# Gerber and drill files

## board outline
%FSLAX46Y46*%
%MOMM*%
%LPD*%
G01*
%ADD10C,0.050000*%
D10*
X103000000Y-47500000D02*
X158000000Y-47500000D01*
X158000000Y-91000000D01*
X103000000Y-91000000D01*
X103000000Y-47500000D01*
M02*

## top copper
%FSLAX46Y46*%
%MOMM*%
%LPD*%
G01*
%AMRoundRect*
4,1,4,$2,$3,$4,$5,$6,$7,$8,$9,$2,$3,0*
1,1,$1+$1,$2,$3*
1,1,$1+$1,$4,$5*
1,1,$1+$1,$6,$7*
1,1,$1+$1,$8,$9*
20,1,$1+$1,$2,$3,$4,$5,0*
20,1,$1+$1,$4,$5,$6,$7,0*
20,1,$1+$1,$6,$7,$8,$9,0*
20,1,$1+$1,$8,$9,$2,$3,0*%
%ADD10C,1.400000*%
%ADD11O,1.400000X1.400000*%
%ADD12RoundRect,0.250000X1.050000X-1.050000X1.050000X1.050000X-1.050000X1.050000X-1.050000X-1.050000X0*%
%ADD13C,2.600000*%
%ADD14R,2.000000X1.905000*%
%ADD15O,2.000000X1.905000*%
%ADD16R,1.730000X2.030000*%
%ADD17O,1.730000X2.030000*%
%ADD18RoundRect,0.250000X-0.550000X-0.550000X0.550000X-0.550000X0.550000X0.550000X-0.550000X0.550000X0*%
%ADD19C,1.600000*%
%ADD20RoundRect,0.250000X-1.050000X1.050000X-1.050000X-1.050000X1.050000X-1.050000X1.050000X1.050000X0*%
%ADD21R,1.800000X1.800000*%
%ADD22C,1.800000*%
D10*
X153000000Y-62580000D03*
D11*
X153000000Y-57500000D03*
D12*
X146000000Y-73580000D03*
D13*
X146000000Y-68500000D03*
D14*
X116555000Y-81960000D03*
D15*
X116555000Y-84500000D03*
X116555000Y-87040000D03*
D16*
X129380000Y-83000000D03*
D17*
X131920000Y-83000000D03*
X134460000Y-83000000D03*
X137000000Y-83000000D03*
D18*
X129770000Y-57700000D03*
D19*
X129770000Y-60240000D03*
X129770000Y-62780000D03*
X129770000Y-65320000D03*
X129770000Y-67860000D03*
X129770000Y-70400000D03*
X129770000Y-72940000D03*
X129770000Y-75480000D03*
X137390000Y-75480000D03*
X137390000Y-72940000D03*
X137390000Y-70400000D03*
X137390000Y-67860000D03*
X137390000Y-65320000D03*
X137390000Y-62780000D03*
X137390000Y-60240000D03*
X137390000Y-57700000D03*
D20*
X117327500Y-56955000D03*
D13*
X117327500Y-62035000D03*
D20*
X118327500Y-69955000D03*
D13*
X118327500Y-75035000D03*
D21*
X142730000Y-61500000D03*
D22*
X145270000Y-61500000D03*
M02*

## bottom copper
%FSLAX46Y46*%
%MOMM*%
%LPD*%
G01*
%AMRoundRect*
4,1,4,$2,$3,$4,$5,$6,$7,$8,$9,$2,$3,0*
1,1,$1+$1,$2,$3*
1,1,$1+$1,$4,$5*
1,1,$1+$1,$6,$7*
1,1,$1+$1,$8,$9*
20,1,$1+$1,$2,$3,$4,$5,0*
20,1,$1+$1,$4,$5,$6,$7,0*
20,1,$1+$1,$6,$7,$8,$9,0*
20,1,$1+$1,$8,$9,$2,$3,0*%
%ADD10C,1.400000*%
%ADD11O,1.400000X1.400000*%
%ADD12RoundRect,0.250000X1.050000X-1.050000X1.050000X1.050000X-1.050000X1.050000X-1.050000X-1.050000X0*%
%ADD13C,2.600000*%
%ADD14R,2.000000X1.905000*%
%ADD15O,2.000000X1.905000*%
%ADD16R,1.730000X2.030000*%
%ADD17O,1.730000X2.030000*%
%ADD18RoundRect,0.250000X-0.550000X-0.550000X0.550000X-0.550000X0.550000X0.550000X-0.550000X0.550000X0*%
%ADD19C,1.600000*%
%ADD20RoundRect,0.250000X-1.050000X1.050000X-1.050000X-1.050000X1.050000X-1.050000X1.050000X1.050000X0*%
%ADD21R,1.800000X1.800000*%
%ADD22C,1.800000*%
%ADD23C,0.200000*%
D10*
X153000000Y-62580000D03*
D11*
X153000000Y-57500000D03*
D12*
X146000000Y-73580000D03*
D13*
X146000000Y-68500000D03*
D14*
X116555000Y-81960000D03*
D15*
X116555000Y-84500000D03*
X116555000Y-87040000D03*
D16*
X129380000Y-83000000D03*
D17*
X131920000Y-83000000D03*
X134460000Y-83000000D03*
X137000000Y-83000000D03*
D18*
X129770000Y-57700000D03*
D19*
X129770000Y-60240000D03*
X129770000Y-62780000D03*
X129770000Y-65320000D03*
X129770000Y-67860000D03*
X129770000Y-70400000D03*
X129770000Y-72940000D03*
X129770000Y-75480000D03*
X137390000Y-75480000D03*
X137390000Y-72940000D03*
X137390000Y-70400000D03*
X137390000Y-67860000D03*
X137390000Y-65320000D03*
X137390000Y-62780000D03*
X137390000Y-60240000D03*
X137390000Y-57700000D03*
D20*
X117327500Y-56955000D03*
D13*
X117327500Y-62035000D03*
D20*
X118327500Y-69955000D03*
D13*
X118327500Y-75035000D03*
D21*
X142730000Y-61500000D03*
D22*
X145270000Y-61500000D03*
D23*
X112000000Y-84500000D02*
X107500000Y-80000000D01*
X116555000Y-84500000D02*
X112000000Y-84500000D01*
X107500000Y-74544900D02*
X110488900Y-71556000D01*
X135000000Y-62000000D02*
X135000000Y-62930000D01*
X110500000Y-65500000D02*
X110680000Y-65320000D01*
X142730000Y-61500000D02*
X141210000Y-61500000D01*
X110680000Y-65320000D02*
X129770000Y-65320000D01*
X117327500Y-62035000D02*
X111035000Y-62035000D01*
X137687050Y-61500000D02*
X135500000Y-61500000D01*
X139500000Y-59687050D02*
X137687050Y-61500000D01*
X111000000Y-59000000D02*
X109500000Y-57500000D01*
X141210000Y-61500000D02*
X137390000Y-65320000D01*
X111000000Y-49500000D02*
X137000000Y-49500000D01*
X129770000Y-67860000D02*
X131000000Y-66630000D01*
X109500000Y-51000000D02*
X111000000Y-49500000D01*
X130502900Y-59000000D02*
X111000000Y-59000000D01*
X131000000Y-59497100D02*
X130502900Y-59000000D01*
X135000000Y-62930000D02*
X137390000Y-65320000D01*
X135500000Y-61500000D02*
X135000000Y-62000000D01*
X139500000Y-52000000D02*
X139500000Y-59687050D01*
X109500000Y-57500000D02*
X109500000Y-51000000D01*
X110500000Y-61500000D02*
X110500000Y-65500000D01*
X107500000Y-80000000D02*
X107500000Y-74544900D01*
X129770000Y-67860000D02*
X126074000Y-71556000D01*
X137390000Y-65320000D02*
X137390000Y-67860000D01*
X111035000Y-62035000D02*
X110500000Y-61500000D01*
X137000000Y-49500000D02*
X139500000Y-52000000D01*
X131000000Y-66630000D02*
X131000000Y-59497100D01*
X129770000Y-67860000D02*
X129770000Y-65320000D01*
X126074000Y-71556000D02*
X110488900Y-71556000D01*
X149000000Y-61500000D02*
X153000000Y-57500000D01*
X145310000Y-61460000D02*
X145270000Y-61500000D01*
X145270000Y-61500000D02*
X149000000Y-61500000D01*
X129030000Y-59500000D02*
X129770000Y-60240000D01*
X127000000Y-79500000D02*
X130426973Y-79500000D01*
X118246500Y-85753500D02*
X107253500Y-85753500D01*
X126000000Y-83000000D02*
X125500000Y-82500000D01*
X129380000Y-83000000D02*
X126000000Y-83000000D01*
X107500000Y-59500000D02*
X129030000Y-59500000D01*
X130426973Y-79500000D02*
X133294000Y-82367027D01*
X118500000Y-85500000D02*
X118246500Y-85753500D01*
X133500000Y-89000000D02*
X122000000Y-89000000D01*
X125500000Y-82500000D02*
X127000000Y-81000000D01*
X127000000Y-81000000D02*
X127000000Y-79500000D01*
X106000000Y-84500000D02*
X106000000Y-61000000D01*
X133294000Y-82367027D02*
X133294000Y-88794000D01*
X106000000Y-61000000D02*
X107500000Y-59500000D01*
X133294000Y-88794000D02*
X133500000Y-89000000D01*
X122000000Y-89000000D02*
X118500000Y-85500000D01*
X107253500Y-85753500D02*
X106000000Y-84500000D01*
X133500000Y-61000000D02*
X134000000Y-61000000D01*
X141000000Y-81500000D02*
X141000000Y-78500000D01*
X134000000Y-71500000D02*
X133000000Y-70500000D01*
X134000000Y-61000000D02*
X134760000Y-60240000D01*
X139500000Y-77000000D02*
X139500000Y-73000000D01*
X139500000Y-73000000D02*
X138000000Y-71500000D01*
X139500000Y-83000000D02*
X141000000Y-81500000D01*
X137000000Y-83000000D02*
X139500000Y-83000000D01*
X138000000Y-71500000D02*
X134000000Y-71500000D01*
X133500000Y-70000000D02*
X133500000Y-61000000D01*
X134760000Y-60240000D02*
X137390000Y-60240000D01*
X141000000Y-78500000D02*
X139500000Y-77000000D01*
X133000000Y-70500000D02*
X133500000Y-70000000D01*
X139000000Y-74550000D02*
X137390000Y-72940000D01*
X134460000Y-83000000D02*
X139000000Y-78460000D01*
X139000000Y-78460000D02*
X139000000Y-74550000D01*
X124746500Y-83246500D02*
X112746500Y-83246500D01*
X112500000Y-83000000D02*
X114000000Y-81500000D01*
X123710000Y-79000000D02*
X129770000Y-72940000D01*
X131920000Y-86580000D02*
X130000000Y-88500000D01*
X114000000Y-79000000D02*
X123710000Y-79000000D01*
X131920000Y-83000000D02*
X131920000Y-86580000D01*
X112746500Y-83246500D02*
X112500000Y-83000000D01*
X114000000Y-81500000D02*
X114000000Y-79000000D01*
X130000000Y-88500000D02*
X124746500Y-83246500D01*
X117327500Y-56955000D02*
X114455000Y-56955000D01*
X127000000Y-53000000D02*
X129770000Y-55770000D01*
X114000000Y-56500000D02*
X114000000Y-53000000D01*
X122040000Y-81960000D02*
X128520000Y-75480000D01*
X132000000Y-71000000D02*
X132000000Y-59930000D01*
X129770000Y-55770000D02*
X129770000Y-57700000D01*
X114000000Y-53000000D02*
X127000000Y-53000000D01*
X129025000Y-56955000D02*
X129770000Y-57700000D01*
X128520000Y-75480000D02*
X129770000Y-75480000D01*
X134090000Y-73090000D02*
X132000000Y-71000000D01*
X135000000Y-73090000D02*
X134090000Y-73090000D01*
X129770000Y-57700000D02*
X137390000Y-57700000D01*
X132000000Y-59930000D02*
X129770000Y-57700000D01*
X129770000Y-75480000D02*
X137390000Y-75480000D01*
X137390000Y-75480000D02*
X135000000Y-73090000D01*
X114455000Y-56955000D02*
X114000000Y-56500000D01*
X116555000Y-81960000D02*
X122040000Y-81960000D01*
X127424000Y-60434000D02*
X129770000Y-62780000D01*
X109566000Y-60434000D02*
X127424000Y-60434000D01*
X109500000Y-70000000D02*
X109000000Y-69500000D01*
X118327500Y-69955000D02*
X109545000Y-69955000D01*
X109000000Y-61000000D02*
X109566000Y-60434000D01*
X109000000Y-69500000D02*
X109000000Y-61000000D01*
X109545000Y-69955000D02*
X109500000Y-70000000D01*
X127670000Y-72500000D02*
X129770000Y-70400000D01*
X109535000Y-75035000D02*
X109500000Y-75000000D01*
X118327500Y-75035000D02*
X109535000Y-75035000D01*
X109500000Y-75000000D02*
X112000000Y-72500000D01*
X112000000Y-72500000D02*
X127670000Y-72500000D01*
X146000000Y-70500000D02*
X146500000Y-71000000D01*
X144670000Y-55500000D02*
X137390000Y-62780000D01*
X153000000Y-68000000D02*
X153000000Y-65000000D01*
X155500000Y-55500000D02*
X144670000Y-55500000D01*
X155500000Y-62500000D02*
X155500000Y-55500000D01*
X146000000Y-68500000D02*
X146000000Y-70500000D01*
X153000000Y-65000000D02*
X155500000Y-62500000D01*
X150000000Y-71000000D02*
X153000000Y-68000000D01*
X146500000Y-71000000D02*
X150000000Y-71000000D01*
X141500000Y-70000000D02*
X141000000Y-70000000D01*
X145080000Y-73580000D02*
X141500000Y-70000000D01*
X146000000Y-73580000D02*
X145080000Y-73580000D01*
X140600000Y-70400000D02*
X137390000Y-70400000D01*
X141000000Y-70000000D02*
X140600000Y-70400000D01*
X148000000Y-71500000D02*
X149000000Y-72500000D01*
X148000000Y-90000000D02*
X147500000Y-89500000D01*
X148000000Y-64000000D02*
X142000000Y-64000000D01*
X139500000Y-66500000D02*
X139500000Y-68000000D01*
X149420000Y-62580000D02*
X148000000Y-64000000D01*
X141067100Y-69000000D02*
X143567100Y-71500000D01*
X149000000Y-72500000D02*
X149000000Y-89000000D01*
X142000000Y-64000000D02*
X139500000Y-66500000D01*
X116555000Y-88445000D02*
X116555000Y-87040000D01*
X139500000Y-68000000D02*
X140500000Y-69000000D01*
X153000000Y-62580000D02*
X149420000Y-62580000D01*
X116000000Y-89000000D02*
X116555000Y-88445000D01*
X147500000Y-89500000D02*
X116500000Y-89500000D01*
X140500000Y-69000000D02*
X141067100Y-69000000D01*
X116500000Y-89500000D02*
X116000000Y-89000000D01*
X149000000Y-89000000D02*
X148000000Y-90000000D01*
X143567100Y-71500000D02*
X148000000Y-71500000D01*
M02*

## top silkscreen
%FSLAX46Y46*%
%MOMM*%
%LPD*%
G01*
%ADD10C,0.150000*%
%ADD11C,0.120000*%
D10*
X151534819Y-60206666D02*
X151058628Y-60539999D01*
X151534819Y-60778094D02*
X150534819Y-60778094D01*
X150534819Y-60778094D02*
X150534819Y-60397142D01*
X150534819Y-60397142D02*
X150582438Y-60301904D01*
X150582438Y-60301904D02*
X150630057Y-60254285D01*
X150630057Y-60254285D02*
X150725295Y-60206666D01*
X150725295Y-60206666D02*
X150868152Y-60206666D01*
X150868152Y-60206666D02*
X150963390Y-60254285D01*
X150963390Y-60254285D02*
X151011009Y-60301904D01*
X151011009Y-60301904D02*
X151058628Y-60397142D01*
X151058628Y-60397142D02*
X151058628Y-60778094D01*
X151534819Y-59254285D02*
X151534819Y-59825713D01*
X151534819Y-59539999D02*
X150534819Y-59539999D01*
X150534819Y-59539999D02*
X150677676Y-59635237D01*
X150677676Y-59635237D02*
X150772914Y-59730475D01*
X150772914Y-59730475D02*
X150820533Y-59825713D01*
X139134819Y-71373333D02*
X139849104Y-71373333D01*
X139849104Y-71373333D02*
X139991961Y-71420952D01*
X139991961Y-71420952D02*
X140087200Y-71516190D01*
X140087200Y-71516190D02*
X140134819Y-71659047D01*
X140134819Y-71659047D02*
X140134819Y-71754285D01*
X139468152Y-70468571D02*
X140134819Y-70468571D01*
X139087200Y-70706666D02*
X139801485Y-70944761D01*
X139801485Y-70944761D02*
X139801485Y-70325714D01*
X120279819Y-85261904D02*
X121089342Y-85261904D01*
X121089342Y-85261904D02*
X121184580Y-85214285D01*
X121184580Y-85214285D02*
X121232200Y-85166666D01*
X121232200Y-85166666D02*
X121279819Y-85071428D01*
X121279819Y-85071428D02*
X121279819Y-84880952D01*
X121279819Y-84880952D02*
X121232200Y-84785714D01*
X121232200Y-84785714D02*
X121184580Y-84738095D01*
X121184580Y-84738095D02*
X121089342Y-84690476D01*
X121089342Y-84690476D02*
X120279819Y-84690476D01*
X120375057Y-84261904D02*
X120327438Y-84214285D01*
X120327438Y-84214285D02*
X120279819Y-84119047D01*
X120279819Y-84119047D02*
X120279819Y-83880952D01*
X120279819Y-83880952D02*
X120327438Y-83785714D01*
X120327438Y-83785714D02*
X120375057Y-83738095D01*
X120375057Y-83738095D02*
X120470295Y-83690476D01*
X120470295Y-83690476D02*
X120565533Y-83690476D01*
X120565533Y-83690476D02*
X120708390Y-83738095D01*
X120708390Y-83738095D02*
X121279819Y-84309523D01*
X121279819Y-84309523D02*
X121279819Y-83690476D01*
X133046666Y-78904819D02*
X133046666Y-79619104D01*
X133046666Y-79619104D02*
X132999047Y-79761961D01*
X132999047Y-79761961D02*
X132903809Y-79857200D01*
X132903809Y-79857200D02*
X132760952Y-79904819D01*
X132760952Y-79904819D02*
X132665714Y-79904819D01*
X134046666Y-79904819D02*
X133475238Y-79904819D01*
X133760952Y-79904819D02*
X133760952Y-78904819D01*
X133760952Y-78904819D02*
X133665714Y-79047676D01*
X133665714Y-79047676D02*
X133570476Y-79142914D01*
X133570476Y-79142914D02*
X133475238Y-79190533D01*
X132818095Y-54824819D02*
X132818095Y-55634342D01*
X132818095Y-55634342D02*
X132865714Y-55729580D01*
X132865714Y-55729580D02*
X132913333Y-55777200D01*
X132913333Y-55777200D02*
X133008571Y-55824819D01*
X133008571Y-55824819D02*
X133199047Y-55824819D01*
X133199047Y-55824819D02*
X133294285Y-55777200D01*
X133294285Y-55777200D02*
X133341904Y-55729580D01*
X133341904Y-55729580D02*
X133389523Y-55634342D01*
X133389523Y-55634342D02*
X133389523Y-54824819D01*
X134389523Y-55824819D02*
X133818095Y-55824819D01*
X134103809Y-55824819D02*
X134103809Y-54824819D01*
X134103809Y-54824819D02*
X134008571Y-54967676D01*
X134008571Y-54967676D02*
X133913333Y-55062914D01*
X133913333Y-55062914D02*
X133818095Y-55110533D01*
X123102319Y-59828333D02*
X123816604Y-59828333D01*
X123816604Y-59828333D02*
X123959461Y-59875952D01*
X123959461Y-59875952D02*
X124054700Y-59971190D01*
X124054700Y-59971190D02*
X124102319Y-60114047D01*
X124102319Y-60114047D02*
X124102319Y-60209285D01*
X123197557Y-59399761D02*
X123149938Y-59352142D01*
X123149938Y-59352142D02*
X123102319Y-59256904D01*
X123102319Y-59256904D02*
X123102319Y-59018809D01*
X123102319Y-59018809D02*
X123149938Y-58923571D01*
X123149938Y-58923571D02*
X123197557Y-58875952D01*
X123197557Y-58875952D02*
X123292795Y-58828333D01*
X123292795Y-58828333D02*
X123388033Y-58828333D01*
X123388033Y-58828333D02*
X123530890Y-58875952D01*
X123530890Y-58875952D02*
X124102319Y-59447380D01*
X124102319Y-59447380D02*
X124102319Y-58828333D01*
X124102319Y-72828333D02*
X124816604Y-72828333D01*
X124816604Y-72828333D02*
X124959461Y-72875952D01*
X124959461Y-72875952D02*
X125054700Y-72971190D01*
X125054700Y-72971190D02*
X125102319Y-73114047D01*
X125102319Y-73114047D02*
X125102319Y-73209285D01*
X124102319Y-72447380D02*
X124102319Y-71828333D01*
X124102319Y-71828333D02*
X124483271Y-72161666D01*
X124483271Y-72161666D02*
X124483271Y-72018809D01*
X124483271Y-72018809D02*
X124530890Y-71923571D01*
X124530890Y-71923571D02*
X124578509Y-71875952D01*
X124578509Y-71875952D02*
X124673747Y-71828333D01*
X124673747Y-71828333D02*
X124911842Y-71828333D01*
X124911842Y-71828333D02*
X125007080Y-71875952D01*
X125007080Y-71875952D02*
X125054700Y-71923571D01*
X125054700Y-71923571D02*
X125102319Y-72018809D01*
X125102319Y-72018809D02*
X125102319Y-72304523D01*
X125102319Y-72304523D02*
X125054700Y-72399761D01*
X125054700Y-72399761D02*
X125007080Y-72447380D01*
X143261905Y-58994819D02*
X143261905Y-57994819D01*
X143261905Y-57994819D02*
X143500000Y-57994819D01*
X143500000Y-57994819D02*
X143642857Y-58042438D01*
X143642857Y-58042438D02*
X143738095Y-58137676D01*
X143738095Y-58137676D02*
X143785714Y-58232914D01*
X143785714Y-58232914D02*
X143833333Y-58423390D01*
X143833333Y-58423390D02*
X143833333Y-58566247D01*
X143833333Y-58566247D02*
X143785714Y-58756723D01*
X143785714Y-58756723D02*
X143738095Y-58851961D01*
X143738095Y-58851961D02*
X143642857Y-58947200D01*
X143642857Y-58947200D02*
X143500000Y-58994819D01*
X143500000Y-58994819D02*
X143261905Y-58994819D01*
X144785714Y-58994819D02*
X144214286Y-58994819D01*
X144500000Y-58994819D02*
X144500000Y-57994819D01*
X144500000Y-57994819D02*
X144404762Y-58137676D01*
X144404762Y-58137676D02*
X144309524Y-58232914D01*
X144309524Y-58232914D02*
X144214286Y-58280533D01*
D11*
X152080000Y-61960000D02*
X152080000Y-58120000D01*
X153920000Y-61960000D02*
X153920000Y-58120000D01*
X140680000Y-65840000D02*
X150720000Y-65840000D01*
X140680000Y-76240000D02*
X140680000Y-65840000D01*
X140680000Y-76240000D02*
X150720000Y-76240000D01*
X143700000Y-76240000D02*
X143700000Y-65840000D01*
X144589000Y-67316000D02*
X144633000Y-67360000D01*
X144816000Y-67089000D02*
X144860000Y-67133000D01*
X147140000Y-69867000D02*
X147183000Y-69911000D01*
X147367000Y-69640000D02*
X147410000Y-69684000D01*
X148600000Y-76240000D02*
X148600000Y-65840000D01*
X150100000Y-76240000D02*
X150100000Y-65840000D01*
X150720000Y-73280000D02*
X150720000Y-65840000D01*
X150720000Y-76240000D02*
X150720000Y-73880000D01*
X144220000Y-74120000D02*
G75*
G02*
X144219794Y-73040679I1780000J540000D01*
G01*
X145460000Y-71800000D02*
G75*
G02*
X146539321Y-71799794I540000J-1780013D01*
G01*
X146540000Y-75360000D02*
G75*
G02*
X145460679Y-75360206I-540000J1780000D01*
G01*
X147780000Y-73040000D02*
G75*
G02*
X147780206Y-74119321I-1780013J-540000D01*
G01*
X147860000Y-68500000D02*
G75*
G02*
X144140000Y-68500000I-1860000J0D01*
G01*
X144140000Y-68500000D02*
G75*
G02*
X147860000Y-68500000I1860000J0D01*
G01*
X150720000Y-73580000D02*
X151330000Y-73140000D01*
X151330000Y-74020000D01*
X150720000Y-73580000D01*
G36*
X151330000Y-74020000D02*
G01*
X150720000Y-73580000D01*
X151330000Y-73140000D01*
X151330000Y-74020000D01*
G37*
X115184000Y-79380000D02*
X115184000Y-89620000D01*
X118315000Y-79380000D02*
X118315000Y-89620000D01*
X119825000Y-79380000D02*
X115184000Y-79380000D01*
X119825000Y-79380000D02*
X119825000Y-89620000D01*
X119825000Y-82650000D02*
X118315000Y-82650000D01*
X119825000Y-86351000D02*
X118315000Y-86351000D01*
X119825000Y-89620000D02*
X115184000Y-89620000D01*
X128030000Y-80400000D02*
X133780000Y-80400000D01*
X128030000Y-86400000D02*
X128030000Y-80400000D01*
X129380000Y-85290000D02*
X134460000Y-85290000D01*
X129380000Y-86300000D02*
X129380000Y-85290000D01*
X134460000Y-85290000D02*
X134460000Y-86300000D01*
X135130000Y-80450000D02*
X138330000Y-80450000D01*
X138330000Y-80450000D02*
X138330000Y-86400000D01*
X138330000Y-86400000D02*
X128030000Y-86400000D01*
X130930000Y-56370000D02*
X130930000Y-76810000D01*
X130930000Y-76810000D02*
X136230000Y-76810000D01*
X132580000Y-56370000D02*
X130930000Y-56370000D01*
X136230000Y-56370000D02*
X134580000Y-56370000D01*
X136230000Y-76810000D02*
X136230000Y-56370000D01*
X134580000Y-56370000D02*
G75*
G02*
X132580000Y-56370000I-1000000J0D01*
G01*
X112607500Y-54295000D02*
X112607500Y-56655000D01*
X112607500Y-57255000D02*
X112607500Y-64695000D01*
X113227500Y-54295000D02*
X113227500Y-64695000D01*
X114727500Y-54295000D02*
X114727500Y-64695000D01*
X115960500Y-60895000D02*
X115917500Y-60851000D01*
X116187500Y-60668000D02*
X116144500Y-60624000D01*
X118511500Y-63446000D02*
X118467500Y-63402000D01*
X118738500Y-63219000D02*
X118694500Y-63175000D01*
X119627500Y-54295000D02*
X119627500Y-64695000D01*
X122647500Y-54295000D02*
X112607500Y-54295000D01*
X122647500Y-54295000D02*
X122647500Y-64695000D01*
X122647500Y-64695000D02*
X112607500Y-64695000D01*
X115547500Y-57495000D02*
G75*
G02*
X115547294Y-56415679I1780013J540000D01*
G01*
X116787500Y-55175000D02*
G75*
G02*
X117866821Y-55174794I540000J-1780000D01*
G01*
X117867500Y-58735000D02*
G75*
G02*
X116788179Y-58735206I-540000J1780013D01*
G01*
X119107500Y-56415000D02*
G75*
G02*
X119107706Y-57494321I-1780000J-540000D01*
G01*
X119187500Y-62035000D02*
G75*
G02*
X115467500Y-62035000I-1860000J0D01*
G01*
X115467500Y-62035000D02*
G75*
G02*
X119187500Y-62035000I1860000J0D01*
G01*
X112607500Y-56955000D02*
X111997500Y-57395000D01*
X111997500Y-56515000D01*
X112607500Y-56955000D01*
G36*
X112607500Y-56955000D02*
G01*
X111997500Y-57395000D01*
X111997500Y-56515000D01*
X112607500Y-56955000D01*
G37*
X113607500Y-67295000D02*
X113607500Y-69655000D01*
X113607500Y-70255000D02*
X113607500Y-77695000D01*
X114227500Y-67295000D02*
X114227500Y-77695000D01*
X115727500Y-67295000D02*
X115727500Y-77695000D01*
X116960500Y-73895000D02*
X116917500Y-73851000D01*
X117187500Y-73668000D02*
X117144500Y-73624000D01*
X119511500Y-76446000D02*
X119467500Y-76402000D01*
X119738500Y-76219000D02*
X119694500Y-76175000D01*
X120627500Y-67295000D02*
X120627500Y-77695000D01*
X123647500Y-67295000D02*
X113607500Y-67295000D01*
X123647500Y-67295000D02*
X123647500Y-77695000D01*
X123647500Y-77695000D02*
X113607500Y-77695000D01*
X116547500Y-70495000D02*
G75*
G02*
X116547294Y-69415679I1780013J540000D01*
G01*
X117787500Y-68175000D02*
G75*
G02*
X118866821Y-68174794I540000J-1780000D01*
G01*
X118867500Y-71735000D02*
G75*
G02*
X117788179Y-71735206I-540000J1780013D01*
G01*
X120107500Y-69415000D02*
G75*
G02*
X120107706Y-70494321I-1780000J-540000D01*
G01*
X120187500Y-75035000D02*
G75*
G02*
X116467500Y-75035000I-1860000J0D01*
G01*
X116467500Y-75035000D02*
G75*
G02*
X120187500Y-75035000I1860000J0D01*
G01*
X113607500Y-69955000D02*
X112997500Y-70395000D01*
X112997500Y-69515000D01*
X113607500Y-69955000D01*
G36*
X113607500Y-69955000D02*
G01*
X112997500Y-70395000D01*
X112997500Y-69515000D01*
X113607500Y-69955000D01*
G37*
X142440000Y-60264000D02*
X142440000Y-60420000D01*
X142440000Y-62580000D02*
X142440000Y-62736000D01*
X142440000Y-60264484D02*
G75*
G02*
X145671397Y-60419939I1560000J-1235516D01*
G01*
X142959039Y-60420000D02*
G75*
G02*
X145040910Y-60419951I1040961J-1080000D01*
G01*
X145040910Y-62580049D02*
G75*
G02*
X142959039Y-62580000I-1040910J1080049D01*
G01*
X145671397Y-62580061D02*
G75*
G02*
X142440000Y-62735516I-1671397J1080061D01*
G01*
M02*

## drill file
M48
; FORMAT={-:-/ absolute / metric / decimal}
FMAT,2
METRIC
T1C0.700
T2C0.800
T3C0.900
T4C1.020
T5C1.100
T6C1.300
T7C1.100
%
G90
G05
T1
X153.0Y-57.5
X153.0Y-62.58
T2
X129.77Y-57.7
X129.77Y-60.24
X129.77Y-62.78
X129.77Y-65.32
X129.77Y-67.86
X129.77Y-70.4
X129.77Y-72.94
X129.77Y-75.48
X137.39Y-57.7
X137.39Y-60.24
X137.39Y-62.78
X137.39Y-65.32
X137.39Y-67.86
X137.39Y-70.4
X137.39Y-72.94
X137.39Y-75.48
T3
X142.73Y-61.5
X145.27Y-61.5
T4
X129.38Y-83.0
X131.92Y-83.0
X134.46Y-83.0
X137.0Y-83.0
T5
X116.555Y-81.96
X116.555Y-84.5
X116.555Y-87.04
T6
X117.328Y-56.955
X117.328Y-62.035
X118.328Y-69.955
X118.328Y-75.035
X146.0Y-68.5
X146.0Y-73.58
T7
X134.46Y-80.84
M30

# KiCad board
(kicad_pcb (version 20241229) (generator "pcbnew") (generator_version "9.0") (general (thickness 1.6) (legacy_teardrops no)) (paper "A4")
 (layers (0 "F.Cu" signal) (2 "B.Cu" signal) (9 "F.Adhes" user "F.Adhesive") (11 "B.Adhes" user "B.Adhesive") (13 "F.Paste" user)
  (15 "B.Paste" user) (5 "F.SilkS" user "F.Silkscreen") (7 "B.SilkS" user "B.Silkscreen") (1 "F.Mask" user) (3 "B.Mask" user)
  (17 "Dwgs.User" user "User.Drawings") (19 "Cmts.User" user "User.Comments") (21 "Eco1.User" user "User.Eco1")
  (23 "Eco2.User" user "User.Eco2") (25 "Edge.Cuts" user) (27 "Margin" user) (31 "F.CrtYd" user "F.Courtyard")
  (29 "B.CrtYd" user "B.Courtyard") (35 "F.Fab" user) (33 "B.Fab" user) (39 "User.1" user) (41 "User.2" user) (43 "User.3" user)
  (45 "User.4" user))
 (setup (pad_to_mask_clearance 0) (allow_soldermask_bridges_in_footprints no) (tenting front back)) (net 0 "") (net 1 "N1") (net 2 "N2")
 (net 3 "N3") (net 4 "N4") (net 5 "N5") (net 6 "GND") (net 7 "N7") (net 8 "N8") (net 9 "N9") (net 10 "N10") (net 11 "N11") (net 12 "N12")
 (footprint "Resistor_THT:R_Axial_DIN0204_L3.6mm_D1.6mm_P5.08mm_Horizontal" (layer "F.Cu") (at 153 62.58 90)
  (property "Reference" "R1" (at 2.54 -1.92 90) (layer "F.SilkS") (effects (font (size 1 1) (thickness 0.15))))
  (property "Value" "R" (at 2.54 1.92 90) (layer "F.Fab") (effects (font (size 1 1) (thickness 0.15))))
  (fp_line (start 0.62 -0.92) (end 4.46 -0.92) (stroke (width 0.12) (type solid)) (layer "F.SilkS"))
  (fp_line (start 0.62 0.92) (end 4.46 0.92) (stroke (width 0.12) (type solid)) (layer "F.SilkS"))
  (pad "1" thru_hole circle (at 0 0 90) (size 1.4 1.4) (drill 0.7) (layers "*.Cu" "*.Mask") (remove_unused_layers no) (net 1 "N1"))
  (pad "2" thru_hole oval (at 5.08 0 90) (size 1.4 1.4) (drill 0.7) (layers "*.Cu" "*.Mask") (remove_unused_layers no) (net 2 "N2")))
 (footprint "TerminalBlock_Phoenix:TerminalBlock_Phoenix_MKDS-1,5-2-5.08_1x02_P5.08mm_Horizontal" (layer "F.Cu") (at 146 73.58 90)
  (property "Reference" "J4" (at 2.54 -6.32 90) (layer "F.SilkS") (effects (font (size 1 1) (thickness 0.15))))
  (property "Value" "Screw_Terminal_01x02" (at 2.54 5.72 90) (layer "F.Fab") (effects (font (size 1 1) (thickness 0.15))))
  (fp_line (start 7.74 -5.32) (end 7.74 4.72) (stroke (width 0.12) (type solid)) (layer "F.SilkS"))
  (fp_line (start -2.66 -5.32) (end 7.74 -5.32) (stroke (width 0.12) (type solid)) (layer "F.SilkS"))
  (fp_line (start -2.66 -5.32) (end -2.66 4.72) (stroke (width 0.12) (type solid)) (layer "F.SilkS"))
  (fp_line (start -2.66 -2.3) (end 7.74 -2.3) (stroke (width 0.12) (type solid)) (layer "F.SilkS"))
  (fp_line (start 6.264 -1.411) (end 6.22 -1.367) (stroke (width 0.12) (type solid)) (layer "F.SilkS"))
  (fp_line (start 6.491 -1.184) (end 6.447 -1.14) (stroke (width 0.12) (type solid)) (layer "F.SilkS"))
  (fp_line (start 3.713 1.14) (end 3.669 1.183) (stroke (width 0.12) (type solid)) (layer "F.SilkS"))
  (fp_line (start 3.94 1.367) (end 3.896 1.41) (stroke (width 0.12) (type solid)) (layer "F.SilkS"))
  (fp_line (start -2.66 2.6) (end 7.74 2.6) (stroke (width 0.12) (type solid)) (layer "F.SilkS"))
  (fp_line (start -2.66 4.1) (end 7.74 4.1) (stroke (width 0.12) (type solid)) (layer "F.SilkS"))
  (fp_line (start 0.3 4.72) (end 7.74 4.72) (stroke (width 0.12) (type solid)) (layer "F.SilkS"))
  (fp_line (start -2.66 4.72) (end -0.3 4.72) (stroke (width 0.12) (type solid)) (layer "F.SilkS"))
  (fp_arc (start -0.54 -1.78) (mid -0.000355 -1.860107) (end 0.539321 -1.780206) (stroke (width 0.12) (type solid)) (layer "F.SilkS"))
  (fp_arc (start 1.78 -0.54) (mid 1.860107 -0.000355) (end 1.780206 0.539321) (stroke (width 0.12) (type solid)) (layer "F.SilkS"))
  (fp_arc (start -1.78 0.54) (mid -1.860107 0.000355) (end -1.780206 -0.539321) (stroke (width 0.12) (type solid)) (layer "F.SilkS"))
  (fp_arc (start 0.54 1.78) (mid 0.000355 1.860107) (end -0.539321 1.780206) (stroke (width 0.12) (type solid)) (layer "F.SilkS"))
  (fp_circle (center 5.08 0) (end 6.94 0) (stroke (width 0.12) (type solid)) (fill no) (layer "F.SilkS"))
  (fp_poly (pts (xy 0 4.72) (xy 0.44 5.33) (xy -0.44 5.33) (xy 0 4.72)) (stroke (width 0.12) (type solid)) (fill yes) (layer "F.SilkS"))
  (pad "1" thru_hole roundrect (at 0 0 90) (size 2.6 2.6) (drill 1.3) (layers "*.Cu" "*.Mask") (remove_unused_layers no)
   (roundrect_rratio 0.096154) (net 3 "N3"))
  (pad "2" thru_hole circle (at 5.08 0 90) (size 2.6 2.6) (drill 1.3) (layers "*.Cu" "*.Mask") (remove_unused_layers no) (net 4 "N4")))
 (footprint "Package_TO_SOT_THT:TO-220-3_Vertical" (layer "F.Cu") (at 116.555 81.96 -90)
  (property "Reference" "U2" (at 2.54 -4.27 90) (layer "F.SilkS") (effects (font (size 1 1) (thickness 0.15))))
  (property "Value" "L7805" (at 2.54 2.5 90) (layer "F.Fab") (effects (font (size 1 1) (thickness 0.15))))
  (fp_line (start -2.58 1.371) (end 7.66 1.371) (stroke (width 0.12) (type solid)) (layer "F.SilkS"))
  (fp_line (start -2.58 -1.76) (end 7.66 -1.76) (stroke (width 0.12) (type solid)) (layer "F.SilkS"))
  (fp_line (start -2.58 -3.27) (end -2.58 1.371) (stroke (width 0.12) (type solid)) (layer "F.SilkS"))
  (fp_line (start -2.58 -3.27) (end 7.66 -3.27) (stroke (width 0.12) (type solid)) (layer "F.SilkS"))
  (fp_line (start 0.69 -3.27) (end 0.69 -1.76) (stroke (width 0.12) (type solid)) (layer "F.SilkS"))
  (fp_line (start 4.391 -3.27) (end 4.391 -1.76) (stroke (width 0.12) (type solid)) (layer "F.SilkS"))
  (fp_line (start 7.66 -3.27) (end 7.66 1.371) (stroke (width 0.12) (type solid)) (layer "F.SilkS"))
  (pad "1" thru_hole rect (at 0 0 270) (size 1.905 2) (drill 1.1) (layers "*.Cu" "*.Mask") (remove_unused_layers no) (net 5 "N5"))
  (pad "2" thru_hole oval (at 2.54 0 270) (size 1.905 2) (drill 1.1) (layers "*.Cu" "*.Mask") (remove_unused_layers no) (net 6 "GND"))
  (pad "3" thru_hole oval (at 5.08 0 270) (size 1.905 2) (drill 1.1) (layers "*.Cu" "*.Mask") (remove_unused_layers no) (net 1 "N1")))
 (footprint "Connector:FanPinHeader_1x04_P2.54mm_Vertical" (layer "F.Cu") (at 129.38 83)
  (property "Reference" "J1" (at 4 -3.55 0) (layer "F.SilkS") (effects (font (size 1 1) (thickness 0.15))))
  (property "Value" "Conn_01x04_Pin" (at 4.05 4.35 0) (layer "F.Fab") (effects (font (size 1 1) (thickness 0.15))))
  (fp_line (start -1.35 -2.6) (end 4.4 -2.6) (stroke (width 0.12) (type solid)) (layer "F.SilkS"))
  (fp_line (start -1.35 3.4) (end -1.35 -2.6) (stroke (width 0.12) (type solid)) (layer "F.SilkS"))
  (fp_line (start 0 2.29) (end 5.08 2.29) (stroke (width 0.12) (type solid)) (layer "F.SilkS"))
  (fp_line (start 0 3.3) (end 0 2.29) (stroke (width 0.12) (type solid)) (layer "F.SilkS"))
  (fp_line (start 5.08 2.29) (end 5.08 3.3) (stroke (width 0.12) (type solid)) (layer "F.SilkS"))
  (fp_line (start 5.75 -2.55) (end 8.95 -2.55) (stroke (width 0.12) (type solid)) (layer "F.SilkS"))
  (fp_line (start 8.95 -2.55) (end 8.95 3.4) (stroke (width 0.12) (type solid)) (layer "F.SilkS"))
  (fp_line (start 8.95 3.4) (end -1.35 3.4) (stroke (width 0.12) (type solid)) (layer "F.SilkS"))
  (pad "" np_thru_hole circle (at 5.08 -2.16 90) (size 1.1 1.1) (drill 1.1) (layers "*.Cu" "*.Mask"))
  (pad "1" thru_hole rect (at 0 0 90) (size 2.03 1.73) (drill 1.02) (layers "*.Cu" "*.Mask") (remove_unused_layers no) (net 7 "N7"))
  (pad "2" thru_hole oval (at 2.54 0 90) (size 2.03 1.73) (drill 1.02) (layers "*.Cu" "*.Mask") (remove_unused_layers no) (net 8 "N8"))
  (pad "3" thru_hole oval (at 5.08 0 90) (size 2.03 1.73) (drill 1.02) (layers "*.Cu" "*.Mask") (remove_unused_layers no) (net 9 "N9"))
  (pad "4" thru_hole oval (at 7.62 0 90) (size 2.03 1.73) (drill 1.02) (layers "*.Cu" "*.Mask") (remove_unused_layers no) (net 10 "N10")))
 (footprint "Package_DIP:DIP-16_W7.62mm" (layer "F.Cu") (at 129.77 57.7)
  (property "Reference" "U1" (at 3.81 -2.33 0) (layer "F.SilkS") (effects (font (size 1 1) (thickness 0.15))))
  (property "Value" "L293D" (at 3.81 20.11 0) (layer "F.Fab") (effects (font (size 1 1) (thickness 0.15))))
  (fp_line (start 1.16 -1.33) (end 1.16 19.11) (stroke (width 0.12) (type solid)) (layer "F.SilkS"))
  (fp_line (start 1.16 19.11) (end 6.46 19.11) (stroke (width 0.12) (type solid)) (layer "F.SilkS"))
  (fp_line (start 2.81 -1.33) (end 1.16 -1.33) (stroke (width 0.12) (type solid)) (layer "F.SilkS"))
  (fp_line (start 6.46 -1.33) (end 4.81 -1.33) (stroke (width 0.12) (type solid)) (layer "F.SilkS"))
  (fp_line (start 6.46 19.11) (end 6.46 -1.33) (stroke (width 0.12) (type solid)) (layer "F.SilkS"))
  (fp_arc (start 4.81 -1.33) (mid 3.81 -0.33) (end 2.81 -1.33) (stroke (width 0.12) (type solid)) (layer "F.SilkS"))
  (pad "1" thru_hole roundrect (at 0 0) (size 1.6 1.6) (drill 0.8) (layers "*.Cu" "*.Mask") (remove_unused_layers no)
   (roundrect_rratio 0.15625) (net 5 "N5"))
  (pad "2" thru_hole circle (at 0 2.54) (size 1.6 1.6) (drill 0.8) (layers "*.Cu" "*.Mask") (remove_unused_layers no) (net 7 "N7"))
  (pad "3" thru_hole circle (at 0 5.08) (size 1.6 1.6) (drill 0.8) (layers "*.Cu" "*.Mask") (remove_unused_layers no) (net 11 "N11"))
  (pad "4" thru_hole circle (at 0 7.62) (size 1.6 1.6) (drill 0.8) (layers "*.Cu" "*.Mask") (remove_unused_layers no) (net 6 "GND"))
  (pad "5" thru_hole circle (at 0 10.16) (size 1.6 1.6) (drill 0.8) (layers "*.Cu" "*.Mask") (remove_unused_layers no) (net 6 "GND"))
  (pad "6" thru_hole circle (at 0 12.7) (size 1.6 1.6) (drill 0.8) (layers "*.Cu" "*.Mask") (remove_unused_layers no) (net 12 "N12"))
  (pad "7" thru_hole circle (at 0 15.24) (size 1.6 1.6) (drill 0.8) (layers "*.Cu" "*.Mask") (remove_unused_layers no) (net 8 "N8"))
  (pad "8" thru_hole circle (at 0 17.78) (size 1.6 1.6) (drill 0.8) (layers "*.Cu" "*.Mask") (remove_unused_layers no) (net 5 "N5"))
  (pad "9" thru_hole circle (at 7.62 17.78) (size 1.6 1.6) (drill 0.8) (layers "*.Cu" "*.Mask") (remove_unused_layers no) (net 5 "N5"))
  (pad "10" thru_hole circle (at 7.62 15.24) (size 1.6 1.6) (drill 0.8) (layers "*.Cu" "*.Mask") (remove_unused_layers no) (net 9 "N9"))
  (pad "11" thru_hole circle (at 7.62 12.7) (size 1.6 1.6) (drill 0.8) (layers "*.Cu" "*.Mask") (remove_unused_layers no) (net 3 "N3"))
  (pad "12" thru_hole circle (at 7.62 10.16) (size 1.6 1.6) (drill 0.8) (layers "*.Cu" "*.Mask") (remove_unused_layers no) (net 6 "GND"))
  (pad "13" thru_hole circle (at 7.62 7.62) (size 1.6 1.6) (drill 0.8) (layers "*.Cu" "*.Mask") (remove_unused_layers no) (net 6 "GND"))
  (pad "14" thru_hole circle (at 7.62 5.08) (size 1.6 1.6) (drill 0.8) (layers "*.Cu" "*.Mask") (remove_unused_layers no) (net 4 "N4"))
  (pad "15" thru_hole circle (at 7.62 2.54) (size 1.6 1.6) (drill 0.8) (layers "*.Cu" "*.Mask") (remove_unused_layers no) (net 10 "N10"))
  (pad "16" thru_hole circle (at 7.62 0) (size 1.6 1.6) (drill 0.8) (layers "*.Cu" "*.Mask") (remove_unused_layers no) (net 5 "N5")))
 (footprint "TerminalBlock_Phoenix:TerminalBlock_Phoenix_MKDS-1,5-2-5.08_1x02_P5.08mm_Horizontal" (layer "F.Cu") (at 117.3275 56.955 -90)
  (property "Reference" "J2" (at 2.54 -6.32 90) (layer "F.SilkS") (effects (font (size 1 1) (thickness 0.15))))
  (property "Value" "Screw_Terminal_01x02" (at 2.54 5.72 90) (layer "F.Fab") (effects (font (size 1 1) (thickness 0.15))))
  (fp_line (start -2.66 4.72) (end -0.3 4.72) (stroke (width 0.12) (type solid)) (layer "F.SilkS"))
  (fp_line (start 0.3 4.72) (end 7.74 4.72) (stroke (width 0.12) (type solid)) (layer "F.SilkS"))
  (fp_line (start -2.66 4.1) (end 7.74 4.1) (stroke (width 0.12) (type solid)) (layer "F.SilkS"))
  (fp_line (start -2.66 2.6) (end 7.74 2.6) (stroke (width 0.12) (type solid)) (layer "F.SilkS"))
  (fp_line (start 3.94 1.367) (end 3.896 1.41) (stroke (width 0.12) (type solid)) (layer "F.SilkS"))
  (fp_line (start 3.713 1.14) (end 3.669 1.183) (stroke (width 0.12) (type solid)) (layer "F.SilkS"))
  (fp_line (start 6.491 -1.184) (end 6.447 -1.14) (stroke (width 0.12) (type solid)) (layer "F.SilkS"))
  (fp_line (start 6.264 -1.411) (end 6.22 -1.367) (stroke (width 0.12) (type solid)) (layer "F.SilkS"))
  (fp_line (start -2.66 -2.3) (end 7.74 -2.3) (stroke (width 0.12) (type solid)) (layer "F.SilkS"))
  (fp_line (start -2.66 -5.32) (end -2.66 4.72) (stroke (width 0.12) (type solid)) (layer "F.SilkS"))
  (fp_line (start -2.66 -5.32) (end 7.74 -5.32) (stroke (width 0.12) (type solid)) (layer "F.SilkS"))
  (fp_line (start 7.74 -5.32) (end 7.74 4.72) (stroke (width 0.12) (type solid)) (layer "F.SilkS"))
  (fp_arc (start 0.54 1.78) (mid 0.000355 1.860107) (end -0.539321 1.780206) (stroke (width 0.12) (type solid)) (layer "F.SilkS"))
  (fp_arc (start -1.78 0.54) (mid -1.860107 0.000355) (end -1.780206 -0.539321) (stroke (width 0.12) (type solid)) (layer "F.SilkS"))
  (fp_arc (start 1.78 -0.54) (mid 1.860107 -0.000355) (end 1.780206 0.539321) (stroke (width 0.12) (type solid)) (layer "F.SilkS"))
  (fp_arc (start -0.54 -1.78) (mid -0.000355 -1.860107) (end 0.539321 -1.780206) (stroke (width 0.12) (type solid)) (layer "F.SilkS"))
  (fp_circle (center 5.08 0) (end 6.94 0) (stroke (width 0.12) (type solid)) (fill no) (layer "F.SilkS"))
  (fp_poly (pts (xy 0 4.72) (xy 0.44 5.33) (xy -0.44 5.33) (xy 0 4.72)) (stroke (width 0.12) (type solid)) (fill yes) (layer "F.SilkS"))
  (pad "1" thru_hole roundrect (at 0 0 270) (size 2.6 2.6) (drill 1.3) (layers "*.Cu" "*.Mask") (remove_unused_layers no)
   (roundrect_rratio 0.096154) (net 5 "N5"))
  (pad "2" thru_hole circle (at 5.08 0 270) (size 2.6 2.6) (drill 1.3) (layers "*.Cu" "*.Mask") (remove_unused_layers no) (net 6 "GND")))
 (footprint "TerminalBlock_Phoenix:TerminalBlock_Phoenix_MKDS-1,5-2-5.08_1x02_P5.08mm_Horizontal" (layer "F.Cu") (at 118.3275 69.955 -90)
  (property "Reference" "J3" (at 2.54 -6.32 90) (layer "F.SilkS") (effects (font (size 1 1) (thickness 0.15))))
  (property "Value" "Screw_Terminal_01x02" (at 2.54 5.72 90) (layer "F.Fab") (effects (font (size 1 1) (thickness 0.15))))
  (fp_line (start -2.66 4.72) (end -0.3 4.72) (stroke (width 0.12) (type solid)) (layer "F.SilkS"))
  (fp_line (start 0.3 4.72) (end 7.74 4.72) (stroke (width 0.12) (type solid)) (layer "F.SilkS"))
  (fp_line (start -2.66 4.1) (end 7.74 4.1) (stroke (width 0.12) (type solid)) (layer "F.SilkS"))
  (fp_line (start -2.66 2.6) (end 7.74 2.6) (stroke (width 0.12) (type solid)) (layer "F.SilkS"))
  (fp_line (start 3.94 1.367) (end 3.896 1.41) (stroke (width 0.12) (type solid)) (layer "F.SilkS"))
  (fp_line (start 3.713 1.14) (end 3.669 1.183) (stroke (width 0.12) (type solid)) (layer "F.SilkS"))
  (fp_line (start 6.491 -1.184) (end 6.447 -1.14) (stroke (width 0.12) (type solid)) (layer "F.SilkS"))
  (fp_line (start 6.264 -1.411) (end 6.22 -1.367) (stroke (width 0.12) (type solid)) (layer "F.SilkS"))
  (fp_line (start -2.66 -2.3) (end 7.74 -2.3) (stroke (width 0.12) (type solid)) (layer "F.SilkS"))
  (fp_line (start -2.66 -5.32) (end -2.66 4.72) (stroke (width 0.12) (type solid)) (layer "F.SilkS"))
  (fp_line (start -2.66 -5.32) (end 7.74 -5.32) (stroke (width 0.12) (type solid)) (layer "F.SilkS"))
  (fp_line (start 7.74 -5.32) (end 7.74 4.72) (stroke (width 0.12) (type solid)) (layer "F.SilkS"))
  (fp_arc (start 0.54 1.78) (mid 0.000355 1.860107) (end -0.539321 1.780206) (stroke (width 0.12) (type solid)) (layer "F.SilkS"))
  (fp_arc (start -1.78 0.54) (mid -1.860107 0.000355) (end -1.780206 -0.539321) (stroke (width 0.12) (type solid)) (layer "F.SilkS"))
  (fp_arc (start 1.78 -0.54) (mid 1.860107 -0.000355) (end 1.780206 0.539321) (stroke (width 0.12) (type solid)) (layer "F.SilkS"))
  (fp_arc (start -0.54 -1.78) (mid -0.000355 -1.860107) (end 0.539321 -1.780206) (stroke (width 0.12) (type solid)) (layer "F.SilkS"))
  (fp_circle (center 5.08 0) (end 6.94 0) (stroke (width 0.12) (type solid)) (fill no) (layer "F.SilkS"))
  (fp_poly (pts (xy 0 4.72) (xy 0.44 5.33) (xy -0.44 5.33) (xy 0 4.72)) (stroke (width 0.12) (type solid)) (fill yes) (layer "F.SilkS"))
  (pad "1" thru_hole roundrect (at 0 0 270) (size 2.6 2.6) (drill 1.3) (layers "*.Cu" "*.Mask") (remove_unused_layers no)
   (roundrect_rratio 0.096154) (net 11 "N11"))
  (pad "2" thru_hole circle (at 5.08 0 270) (size 2.6 2.6) (drill 1.3) (layers "*.Cu" "*.Mask") (remove_unused_layers no) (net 12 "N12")))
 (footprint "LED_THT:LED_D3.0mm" (layer "F.Cu") (at 142.73 61.5)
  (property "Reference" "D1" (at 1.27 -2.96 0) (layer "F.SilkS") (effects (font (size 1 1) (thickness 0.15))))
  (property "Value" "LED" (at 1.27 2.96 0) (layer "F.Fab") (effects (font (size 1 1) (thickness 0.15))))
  (fp_line (start -0.29 -1.236) (end -0.29 -1.08) (stroke (width 0.12) (type solid)) (layer "F.SilkS"))
  (fp_line (start -0.29 1.08) (end -0.29 1.236) (stroke (width 0.12) (type solid)) (layer "F.SilkS"))
  (fp_arc (start -0.29 -1.235516) (mid 1.365624 -1.987701) (end 2.941397 -1.080061) (stroke (width 0.12) (type solid)) (layer "F.SilkS"))
  (fp_arc (start 0.229039 -1.08) (mid 1.269964 -1.5) (end 2.31091 -1.080049) (stroke (width 0.12) (type solid)) (layer "F.SilkS"))
  (fp_arc (start 2.31091 1.080049) (mid 1.269964 1.5) (end 0.229039 1.08) (stroke (width 0.12) (type solid)) (layer "F.SilkS"))
  (fp_arc (start 2.941397 1.080061) (mid 1.365624 1.987701) (end -0.29 1.235516) (stroke (width 0.12) (type solid)) (layer "F.SilkS"))
  (pad "1" thru_hole rect (at 0 0) (size 1.8 1.8) (drill 0.9) (layers "*.Cu" "*.Mask") (remove_unused_layers no) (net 6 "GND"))
  (pad "2" thru_hole circle (at 2.54 0) (size 1.8 1.8) (drill 0.9) (layers "*.Cu" "*.Mask") (remove_unused_layers no) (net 2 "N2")))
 (gr_rect (start 103 47.5) (end 158 91) (stroke (width 0.05) (type default)) (fill no) (layer "Edge.Cuts"))
 (segment (start 112 84.5) (end 107.5 80) (width 0.2) (layer "B.Cu") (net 6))
 (segment (start 116.555 84.5) (end 112 84.5) (width 0.2) (layer "B.Cu") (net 6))
 (segment (start 107.5 74.5449) (end 110.4889 71.556) (width 0.2) (layer "B.Cu") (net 6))
 (segment (start 135 62) (end 135 62.93) (width 0.2) (layer "B.Cu") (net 6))
 (segment (start 110.5 65.5) (end 110.68 65.32) (width 0.2) (layer "B.Cu") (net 6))
 (segment (start 142.73 61.5) (end 141.21 61.5) (width 0.2) (layer "B.Cu") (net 6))
 (segment (start 110.68 65.32) (end 129.77 65.32) (width 0.2) (layer "B.Cu") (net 6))
 (segment (start 117.3275 62.035) (end 111.035 62.035) (width 0.2) (layer "B.Cu") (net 6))
 (segment (start 137.68705 61.5) (end 135.5 61.5) (width 0.2) (layer "B.Cu") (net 6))
 (segment (start 139.5 59.68705) (end 137.68705 61.5) (width 0.2) (layer "B.Cu") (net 6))
 (segment (start 111 59) (end 109.5 57.5) (width 0.2) (layer "B.Cu") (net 6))
 (segment (start 141.21 61.5) (end 137.39 65.32) (width 0.2) (layer "B.Cu") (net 6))
 (segment (start 111 49.5) (end 137 49.5) (width 0.2) (layer "B.Cu") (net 6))
 (segment (start 129.77 67.86) (end 131 66.63) (width 0.2) (layer "B.Cu") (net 6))
 (segment (start 109.5 51) (end 111 49.5) (width 0.2) (layer "B.Cu") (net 6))
 (segment (start 130.5029 59) (end 111 59) (width 0.2) (layer "B.Cu") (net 6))
 (segment (start 131 59.4971) (end 130.5029 59) (width 0.2) (layer "B.Cu") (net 6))
 (segment (start 135 62.93) (end 137.39 65.32) (width 0.2) (layer "B.Cu") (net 6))
 (segment (start 135.5 61.5) (end 135 62) (width 0.2) (layer "B.Cu") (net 6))
 (segment (start 139.5 52) (end 139.5 59.68705) (width 0.2) (layer "B.Cu") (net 6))
 (segment (start 109.5 57.5) (end 109.5 51) (width 0.2) (layer "B.Cu") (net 6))
 (segment (start 110.5 61.5) (end 110.5 65.5) (width 0.2) (layer "B.Cu") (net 6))
 (segment (start 107.5 80) (end 107.5 74.5449) (width 0.2) (layer "B.Cu") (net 6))
 (segment (start 129.77 67.86) (end 126.074 71.556) (width 0.2) (layer "B.Cu") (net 6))
 (segment (start 137.39 65.32) (end 137.39 67.86) (width 0.2) (layer "B.Cu") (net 6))
 (segment (start 111.035 62.035) (end 110.5 61.5) (width 0.2) (layer "B.Cu") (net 6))
 (segment (start 137 49.5) (end 139.5 52) (width 0.2) (layer "B.Cu") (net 6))
 (segment (start 131 66.63) (end 131 59.4971) (width 0.2) (layer "B.Cu") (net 6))
 (segment (start 129.77 67.86) (end 129.77 65.32) (width 0.2) (layer "B.Cu") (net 6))
 (segment (start 126.074 71.556) (end 110.4889 71.556) (width 0.2) (layer "B.Cu") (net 6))
 (segment (start 149 61.5) (end 153 57.5) (width 0.2) (layer "B.Cu") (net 2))
 (segment (start 145.31 61.46) (end 145.27 61.5) (width 0.2) (layer "B.Cu") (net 2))
 (segment (start 145.27 61.5) (end 149 61.5) (width 0.2) (layer "B.Cu") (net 2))
 (segment (start 129.03 59.5) (end 129.77 60.24) (width 0.2) (layer "B.Cu") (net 7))
 (segment (start 127 79.5) (end 130.426973 79.5) (width 0.2) (layer "B.Cu") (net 7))
 (segment (start 118.2465 85.7535) (end 107.2535 85.7535) (width 0.2) (layer "B.Cu") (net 7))
 (segment (start 126 83) (end 125.5 82.5) (width 0.2) (layer "B.Cu") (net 7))
 (segment (start 129.38 83) (end 126 83) (width 0.2) (layer "B.Cu") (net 7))
 (segment (start 107.5 59.5) (end 129.03 59.5) (width 0.2) (layer "B.Cu") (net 7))
 (segment (start 130.426973 79.5) (end 133.294 82.367027) (width 0.2) (layer "B.Cu") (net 7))
 (segment (start 118.5 85.5) (end 118.2465 85.7535) (width 0.2) (layer "B.Cu") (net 7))
 (segment (start 133.5 89) (end 122 89) (width 0.2) (layer "B.Cu") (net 7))
 (segment (start 125.5 82.5) (end 127 81) (width 0.2) (layer "B.Cu") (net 7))
 (segment (start 127 81) (end 127 79.5) (width 0.2) (layer "B.Cu") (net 7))
 (segment (start 106 84.5) (end 106 61) (width 0.2) (layer "B.Cu") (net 7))
 (segment (start 133.294 82.367027) (end 133.294 88.794) (width 0.2) (layer "B.Cu") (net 7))
 (segment (start 106 61) (end 107.5 59.5) (width 0.2) (layer "B.Cu") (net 7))
 (segment (start 133.294 88.794) (end 133.5 89) (width 0.2) (layer "B.Cu") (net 7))
 (segment (start 122 89) (end 118.5 85.5) (width 0.2) (layer "B.Cu") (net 7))
 (segment (start 107.2535 85.7535) (end 106 84.5) (width 0.2) (layer "B.Cu") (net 7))
 (segment (start 133.5 61) (end 134 61) (width 0.2) (layer "B.Cu") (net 10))
 (segment (start 141 81.5) (end 141 78.5) (width 0.2) (layer "B.Cu") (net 10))
 (segment (start 134 71.5) (end 133 70.5) (width 0.2) (layer "B.Cu") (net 10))
 (segment (start 134 61) (end 134.76 60.24) (width 0.2) (layer "B.Cu") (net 10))
 (segment (start 139.5 77) (end 139.5 73) (width 0.2) (layer "B.Cu") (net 10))
 (segment (start 139.5 73) (end 138 71.5) (width 0.2) (layer "B.Cu") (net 10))
 (segment (start 139.5 83) (end 141 81.5) (width 0.2) (layer "B.Cu") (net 10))
 (segment (start 137 83) (end 139.5 83) (width 0.2) (layer "B.Cu") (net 10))
 (segment (start 138 71.5) (end 134 71.5) (width 0.2) (layer "B.Cu") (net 10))
 (segment (start 133.5 70) (end 133.5 61) (width 0.2) (layer "B.Cu") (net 10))
 (segment (start 134.76 60.24) (end 137.39 60.24) (width 0.2) (layer "B.Cu") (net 10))
 (segment (start 141 78.5) (end 139.5 77) (width 0.2) (layer "B.Cu") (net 10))
 (segment (start 133 70.5) (end 133.5 70) (width 0.2) (layer "B.Cu") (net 10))
 (segment (start 139 74.55) (end 137.39 72.94) (width 0.2) (layer "B.Cu") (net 9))
 (segment (start 134.46 83) (end 139 78.46) (width 0.2) (layer "B.Cu") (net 9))
 (segment (start 139 78.46) (end 139 74.55) (width 0.2) (layer "B.Cu") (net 9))
 (segment (start 124.7465 83.2465) (end 112.7465 83.2465) (width 0.2) (layer "B.Cu") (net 8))
 (segment (start 112.5 83) (end 114 81.5) (width 0.2) (layer "B.Cu") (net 8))
 (segment (start 123.71 79) (end 129.77 72.94) (width 0.2) (layer "B.Cu") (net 8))
 (segment (start 131.92 86.58) (end 130 88.5) (width 0.2) (layer "B.Cu") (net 8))
 (segment (start 114 79) (end 123.71 79) (width 0.2) (layer "B.Cu") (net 8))
 (segment (start 131.92 83) (end 131.92 86.58) (width 0.2) (layer "B.Cu") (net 8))
 (segment (start 112.7465 83.2465) (end 112.5 83) (width 0.2) (layer "B.Cu") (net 8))
 (segment (start 114 81.5) (end 114 79) (width 0.2) (layer "B.Cu") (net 8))
 (segment (start 130 88.5) (end 124.7465 83.2465) (width 0.2) (layer "B.Cu") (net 8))
 (segment (start 117.3275 56.955) (end 114.455 56.955) (width 0.2) (layer "B.Cu") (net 5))
 (segment (start 127 53) (end 129.77 55.77) (width 0.2) (layer "B.Cu") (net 5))
 (segment (start 114 56.5) (end 114 53) (width 0.2) (layer "B.Cu") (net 5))
 (segment (start 122.04 81.96) (end 128.52 75.48) (width 0.2) (layer "B.Cu") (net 5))
 (segment (start 132 71) (end 132 59.93) (width 0.2) (layer "B.Cu") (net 5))
 (segment (start 129.77 55.77) (end 129.77 57.7) (width 0.2) (layer "B.Cu") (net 5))
 (segment (start 114 53) (end 127 53) (width 0.2) (layer "B.Cu") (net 5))
 (segment (start 129.025 56.955) (end 129.77 57.7) (width 0.2) (layer "B.Cu") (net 5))
 (segment (start 128.52 75.48) (end 129.77 75.48) (width 0.2) (layer "B.Cu") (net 5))
 (segment (start 134.09 73.09) (end 132 71) (width 0.2) (layer "B.Cu") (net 5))
 (segment (start 135 73.09) (end 134.09 73.09) (width 0.2) (layer "B.Cu") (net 5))
 (segment (start 129.77 57.7) (end 137.39 57.7) (width 0.2) (layer "B.Cu") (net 5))
 (segment (start 132 59.93) (end 129.77 57.7) (width 0.2) (layer "B.Cu") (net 5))
 (segment (start 129.77 75.48) (end 137.39 75.48) (width 0.2) (layer "B.Cu") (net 5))
 (segment (start 137.39 75.48) (end 135 73.09) (width 0.2) (layer "B.Cu") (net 5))
 (segment (start 114.455 56.955) (end 114 56.5) (width 0.2) (layer "B.Cu") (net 5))
 (segment (start 116.555 81.96) (end 122.04 81.96) (width 0.2) (layer "B.Cu") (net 5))
 (segment (start 127.424 60.434) (end 129.77 62.78) (width 0.2) (layer "B.Cu") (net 11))
 (segment (start 109.566 60.434) (end 127.424 60.434) (width 0.2) (layer "B.Cu") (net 11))
 (segment (start 109.5 70) (end 109 69.5) (width 0.2) (layer "B.Cu") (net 11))
 (segment (start 118.3275 69.955) (end 109.545 69.955) (width 0.2) (layer "B.Cu") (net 11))
 (segment (start 109 61) (end 109.566 60.434) (width 0.2) (layer "B.Cu") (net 11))
 (segment (start 109 69.5) (end 109 61) (width 0.2) (layer "B.Cu") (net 11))
 (segment (start 109.545 69.955) (end 109.5 70) (width 0.2) (layer "B.Cu") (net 11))
 (segment (start 127.67 72.5) (end 129.77 70.4) (width 0.2) (layer "B.Cu") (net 12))
 (segment (start 109.535 75.035) (end 109.5 75) (width 0.2) (layer "B.Cu") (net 12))
 (segment (start 118.3275 75.035) (end 109.535 75.035) (width 0.2) (layer "B.Cu") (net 12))
 (segment (start 109.5 75) (end 112 72.5) (width 0.2) (layer "B.Cu") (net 12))
 (segment (start 112 72.5) (end 127.67 72.5) (width 0.2) (layer "B.Cu") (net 12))
 (segment (start 146 70.5) (end 146.5 71) (width 0.2) (layer "B.Cu") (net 4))
 (segment (start 144.67 55.5) (end 137.39 62.78) (width 0.2) (layer "B.Cu") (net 4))
 (segment (start 153 68) (end 153 65) (width 0.2) (layer "B.Cu") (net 4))
 (segment (start 155.5 55.5) (end 144.67 55.5) (width 0.2) (layer "B.Cu") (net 4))
 (segment (start 155.5 62.5) (end 155.5 55.5) (width 0.2) (layer "B.Cu") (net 4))
 (segment (start 146 68.5) (end 146 70.5) (width 0.2) (layer "B.Cu") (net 4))
 (segment (start 153 65) (end 155.5 62.5) (width 0.2) (layer "B.Cu") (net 4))
 (segment (start 150 71) (end 153 68) (width 0.2) (layer "B.Cu") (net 4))
 (segment (start 146.5 71) (end 150 71) (width 0.2) (layer "B.Cu") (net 4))
 (segment (start 141.5 70) (end 141 70) (width 0.2) (layer "B.Cu") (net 3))
 (segment (start 145.08 73.58) (end 141.5 70) (width 0.2) (layer "B.Cu") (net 3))
 (segment (start 146 73.58) (end 145.08 73.58) (width 0.2) (layer "B.Cu") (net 3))
 (segment (start 140.6 70.4) (end 137.39 70.4) (width 0.2) (layer "B.Cu") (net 3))
 (segment (start 141 70) (end 140.6 70.4) (width 0.2) (layer "B.Cu") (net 3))
 (segment (start 148 71.5) (end 149 72.5) (width 0.2) (layer "B.Cu") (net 1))
 (segment (start 148 90) (end 147.5 89.5) (width 0.2) (layer "B.Cu") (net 1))
 (segment (start 148 64) (end 142 64) (width 0.2) (layer "B.Cu") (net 1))
 (segment (start 139.5 66.5) (end 139.5 68) (width 0.2) (layer "B.Cu") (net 1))
 (segment (start 149.42 62.58) (end 148 64) (width 0.2) (layer "B.Cu") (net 1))
 (segment (start 141.0671 69) (end 143.5671 71.5) (width 0.2) (layer "B.Cu") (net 1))
 (segment (start 149 72.5) (end 149 89) (width 0.2) (layer "B.Cu") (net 1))
 (segment (start 142 64) (end 139.5 66.5) (width 0.2) (layer "B.Cu") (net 1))
 (segment (start 116.555 88.445) (end 116.555 87.04) (width 0.2) (layer "B.Cu") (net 1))
 (segment (start 139.5 68) (end 140.5 69) (width 0.2) (layer "B.Cu") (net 1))
 (segment (start 153 62.58) (end 149.42 62.58) (width 0.2) (layer "B.Cu") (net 1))
 (segment (start 116 89) (end 116.555 88.445) (width 0.2) (layer "B.Cu") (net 1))
 (segment (start 147.5 89.5) (end 116.5 89.5) (width 0.2) (layer "B.Cu") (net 1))
 (segment (start 140.5 69) (end 141.0671 69) (width 0.2) (layer "B.Cu") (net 1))
 (segment (start 116.5 89.5) (end 116 89) (width 0.2) (layer "B.Cu") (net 1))
 (segment (start 149 89) (end 148 90) (width 0.2) (layer "B.Cu") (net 1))
 (segment (start 143.5671 71.5) (end 148 71.5) (width 0.2) (layer "B.Cu") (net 1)))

